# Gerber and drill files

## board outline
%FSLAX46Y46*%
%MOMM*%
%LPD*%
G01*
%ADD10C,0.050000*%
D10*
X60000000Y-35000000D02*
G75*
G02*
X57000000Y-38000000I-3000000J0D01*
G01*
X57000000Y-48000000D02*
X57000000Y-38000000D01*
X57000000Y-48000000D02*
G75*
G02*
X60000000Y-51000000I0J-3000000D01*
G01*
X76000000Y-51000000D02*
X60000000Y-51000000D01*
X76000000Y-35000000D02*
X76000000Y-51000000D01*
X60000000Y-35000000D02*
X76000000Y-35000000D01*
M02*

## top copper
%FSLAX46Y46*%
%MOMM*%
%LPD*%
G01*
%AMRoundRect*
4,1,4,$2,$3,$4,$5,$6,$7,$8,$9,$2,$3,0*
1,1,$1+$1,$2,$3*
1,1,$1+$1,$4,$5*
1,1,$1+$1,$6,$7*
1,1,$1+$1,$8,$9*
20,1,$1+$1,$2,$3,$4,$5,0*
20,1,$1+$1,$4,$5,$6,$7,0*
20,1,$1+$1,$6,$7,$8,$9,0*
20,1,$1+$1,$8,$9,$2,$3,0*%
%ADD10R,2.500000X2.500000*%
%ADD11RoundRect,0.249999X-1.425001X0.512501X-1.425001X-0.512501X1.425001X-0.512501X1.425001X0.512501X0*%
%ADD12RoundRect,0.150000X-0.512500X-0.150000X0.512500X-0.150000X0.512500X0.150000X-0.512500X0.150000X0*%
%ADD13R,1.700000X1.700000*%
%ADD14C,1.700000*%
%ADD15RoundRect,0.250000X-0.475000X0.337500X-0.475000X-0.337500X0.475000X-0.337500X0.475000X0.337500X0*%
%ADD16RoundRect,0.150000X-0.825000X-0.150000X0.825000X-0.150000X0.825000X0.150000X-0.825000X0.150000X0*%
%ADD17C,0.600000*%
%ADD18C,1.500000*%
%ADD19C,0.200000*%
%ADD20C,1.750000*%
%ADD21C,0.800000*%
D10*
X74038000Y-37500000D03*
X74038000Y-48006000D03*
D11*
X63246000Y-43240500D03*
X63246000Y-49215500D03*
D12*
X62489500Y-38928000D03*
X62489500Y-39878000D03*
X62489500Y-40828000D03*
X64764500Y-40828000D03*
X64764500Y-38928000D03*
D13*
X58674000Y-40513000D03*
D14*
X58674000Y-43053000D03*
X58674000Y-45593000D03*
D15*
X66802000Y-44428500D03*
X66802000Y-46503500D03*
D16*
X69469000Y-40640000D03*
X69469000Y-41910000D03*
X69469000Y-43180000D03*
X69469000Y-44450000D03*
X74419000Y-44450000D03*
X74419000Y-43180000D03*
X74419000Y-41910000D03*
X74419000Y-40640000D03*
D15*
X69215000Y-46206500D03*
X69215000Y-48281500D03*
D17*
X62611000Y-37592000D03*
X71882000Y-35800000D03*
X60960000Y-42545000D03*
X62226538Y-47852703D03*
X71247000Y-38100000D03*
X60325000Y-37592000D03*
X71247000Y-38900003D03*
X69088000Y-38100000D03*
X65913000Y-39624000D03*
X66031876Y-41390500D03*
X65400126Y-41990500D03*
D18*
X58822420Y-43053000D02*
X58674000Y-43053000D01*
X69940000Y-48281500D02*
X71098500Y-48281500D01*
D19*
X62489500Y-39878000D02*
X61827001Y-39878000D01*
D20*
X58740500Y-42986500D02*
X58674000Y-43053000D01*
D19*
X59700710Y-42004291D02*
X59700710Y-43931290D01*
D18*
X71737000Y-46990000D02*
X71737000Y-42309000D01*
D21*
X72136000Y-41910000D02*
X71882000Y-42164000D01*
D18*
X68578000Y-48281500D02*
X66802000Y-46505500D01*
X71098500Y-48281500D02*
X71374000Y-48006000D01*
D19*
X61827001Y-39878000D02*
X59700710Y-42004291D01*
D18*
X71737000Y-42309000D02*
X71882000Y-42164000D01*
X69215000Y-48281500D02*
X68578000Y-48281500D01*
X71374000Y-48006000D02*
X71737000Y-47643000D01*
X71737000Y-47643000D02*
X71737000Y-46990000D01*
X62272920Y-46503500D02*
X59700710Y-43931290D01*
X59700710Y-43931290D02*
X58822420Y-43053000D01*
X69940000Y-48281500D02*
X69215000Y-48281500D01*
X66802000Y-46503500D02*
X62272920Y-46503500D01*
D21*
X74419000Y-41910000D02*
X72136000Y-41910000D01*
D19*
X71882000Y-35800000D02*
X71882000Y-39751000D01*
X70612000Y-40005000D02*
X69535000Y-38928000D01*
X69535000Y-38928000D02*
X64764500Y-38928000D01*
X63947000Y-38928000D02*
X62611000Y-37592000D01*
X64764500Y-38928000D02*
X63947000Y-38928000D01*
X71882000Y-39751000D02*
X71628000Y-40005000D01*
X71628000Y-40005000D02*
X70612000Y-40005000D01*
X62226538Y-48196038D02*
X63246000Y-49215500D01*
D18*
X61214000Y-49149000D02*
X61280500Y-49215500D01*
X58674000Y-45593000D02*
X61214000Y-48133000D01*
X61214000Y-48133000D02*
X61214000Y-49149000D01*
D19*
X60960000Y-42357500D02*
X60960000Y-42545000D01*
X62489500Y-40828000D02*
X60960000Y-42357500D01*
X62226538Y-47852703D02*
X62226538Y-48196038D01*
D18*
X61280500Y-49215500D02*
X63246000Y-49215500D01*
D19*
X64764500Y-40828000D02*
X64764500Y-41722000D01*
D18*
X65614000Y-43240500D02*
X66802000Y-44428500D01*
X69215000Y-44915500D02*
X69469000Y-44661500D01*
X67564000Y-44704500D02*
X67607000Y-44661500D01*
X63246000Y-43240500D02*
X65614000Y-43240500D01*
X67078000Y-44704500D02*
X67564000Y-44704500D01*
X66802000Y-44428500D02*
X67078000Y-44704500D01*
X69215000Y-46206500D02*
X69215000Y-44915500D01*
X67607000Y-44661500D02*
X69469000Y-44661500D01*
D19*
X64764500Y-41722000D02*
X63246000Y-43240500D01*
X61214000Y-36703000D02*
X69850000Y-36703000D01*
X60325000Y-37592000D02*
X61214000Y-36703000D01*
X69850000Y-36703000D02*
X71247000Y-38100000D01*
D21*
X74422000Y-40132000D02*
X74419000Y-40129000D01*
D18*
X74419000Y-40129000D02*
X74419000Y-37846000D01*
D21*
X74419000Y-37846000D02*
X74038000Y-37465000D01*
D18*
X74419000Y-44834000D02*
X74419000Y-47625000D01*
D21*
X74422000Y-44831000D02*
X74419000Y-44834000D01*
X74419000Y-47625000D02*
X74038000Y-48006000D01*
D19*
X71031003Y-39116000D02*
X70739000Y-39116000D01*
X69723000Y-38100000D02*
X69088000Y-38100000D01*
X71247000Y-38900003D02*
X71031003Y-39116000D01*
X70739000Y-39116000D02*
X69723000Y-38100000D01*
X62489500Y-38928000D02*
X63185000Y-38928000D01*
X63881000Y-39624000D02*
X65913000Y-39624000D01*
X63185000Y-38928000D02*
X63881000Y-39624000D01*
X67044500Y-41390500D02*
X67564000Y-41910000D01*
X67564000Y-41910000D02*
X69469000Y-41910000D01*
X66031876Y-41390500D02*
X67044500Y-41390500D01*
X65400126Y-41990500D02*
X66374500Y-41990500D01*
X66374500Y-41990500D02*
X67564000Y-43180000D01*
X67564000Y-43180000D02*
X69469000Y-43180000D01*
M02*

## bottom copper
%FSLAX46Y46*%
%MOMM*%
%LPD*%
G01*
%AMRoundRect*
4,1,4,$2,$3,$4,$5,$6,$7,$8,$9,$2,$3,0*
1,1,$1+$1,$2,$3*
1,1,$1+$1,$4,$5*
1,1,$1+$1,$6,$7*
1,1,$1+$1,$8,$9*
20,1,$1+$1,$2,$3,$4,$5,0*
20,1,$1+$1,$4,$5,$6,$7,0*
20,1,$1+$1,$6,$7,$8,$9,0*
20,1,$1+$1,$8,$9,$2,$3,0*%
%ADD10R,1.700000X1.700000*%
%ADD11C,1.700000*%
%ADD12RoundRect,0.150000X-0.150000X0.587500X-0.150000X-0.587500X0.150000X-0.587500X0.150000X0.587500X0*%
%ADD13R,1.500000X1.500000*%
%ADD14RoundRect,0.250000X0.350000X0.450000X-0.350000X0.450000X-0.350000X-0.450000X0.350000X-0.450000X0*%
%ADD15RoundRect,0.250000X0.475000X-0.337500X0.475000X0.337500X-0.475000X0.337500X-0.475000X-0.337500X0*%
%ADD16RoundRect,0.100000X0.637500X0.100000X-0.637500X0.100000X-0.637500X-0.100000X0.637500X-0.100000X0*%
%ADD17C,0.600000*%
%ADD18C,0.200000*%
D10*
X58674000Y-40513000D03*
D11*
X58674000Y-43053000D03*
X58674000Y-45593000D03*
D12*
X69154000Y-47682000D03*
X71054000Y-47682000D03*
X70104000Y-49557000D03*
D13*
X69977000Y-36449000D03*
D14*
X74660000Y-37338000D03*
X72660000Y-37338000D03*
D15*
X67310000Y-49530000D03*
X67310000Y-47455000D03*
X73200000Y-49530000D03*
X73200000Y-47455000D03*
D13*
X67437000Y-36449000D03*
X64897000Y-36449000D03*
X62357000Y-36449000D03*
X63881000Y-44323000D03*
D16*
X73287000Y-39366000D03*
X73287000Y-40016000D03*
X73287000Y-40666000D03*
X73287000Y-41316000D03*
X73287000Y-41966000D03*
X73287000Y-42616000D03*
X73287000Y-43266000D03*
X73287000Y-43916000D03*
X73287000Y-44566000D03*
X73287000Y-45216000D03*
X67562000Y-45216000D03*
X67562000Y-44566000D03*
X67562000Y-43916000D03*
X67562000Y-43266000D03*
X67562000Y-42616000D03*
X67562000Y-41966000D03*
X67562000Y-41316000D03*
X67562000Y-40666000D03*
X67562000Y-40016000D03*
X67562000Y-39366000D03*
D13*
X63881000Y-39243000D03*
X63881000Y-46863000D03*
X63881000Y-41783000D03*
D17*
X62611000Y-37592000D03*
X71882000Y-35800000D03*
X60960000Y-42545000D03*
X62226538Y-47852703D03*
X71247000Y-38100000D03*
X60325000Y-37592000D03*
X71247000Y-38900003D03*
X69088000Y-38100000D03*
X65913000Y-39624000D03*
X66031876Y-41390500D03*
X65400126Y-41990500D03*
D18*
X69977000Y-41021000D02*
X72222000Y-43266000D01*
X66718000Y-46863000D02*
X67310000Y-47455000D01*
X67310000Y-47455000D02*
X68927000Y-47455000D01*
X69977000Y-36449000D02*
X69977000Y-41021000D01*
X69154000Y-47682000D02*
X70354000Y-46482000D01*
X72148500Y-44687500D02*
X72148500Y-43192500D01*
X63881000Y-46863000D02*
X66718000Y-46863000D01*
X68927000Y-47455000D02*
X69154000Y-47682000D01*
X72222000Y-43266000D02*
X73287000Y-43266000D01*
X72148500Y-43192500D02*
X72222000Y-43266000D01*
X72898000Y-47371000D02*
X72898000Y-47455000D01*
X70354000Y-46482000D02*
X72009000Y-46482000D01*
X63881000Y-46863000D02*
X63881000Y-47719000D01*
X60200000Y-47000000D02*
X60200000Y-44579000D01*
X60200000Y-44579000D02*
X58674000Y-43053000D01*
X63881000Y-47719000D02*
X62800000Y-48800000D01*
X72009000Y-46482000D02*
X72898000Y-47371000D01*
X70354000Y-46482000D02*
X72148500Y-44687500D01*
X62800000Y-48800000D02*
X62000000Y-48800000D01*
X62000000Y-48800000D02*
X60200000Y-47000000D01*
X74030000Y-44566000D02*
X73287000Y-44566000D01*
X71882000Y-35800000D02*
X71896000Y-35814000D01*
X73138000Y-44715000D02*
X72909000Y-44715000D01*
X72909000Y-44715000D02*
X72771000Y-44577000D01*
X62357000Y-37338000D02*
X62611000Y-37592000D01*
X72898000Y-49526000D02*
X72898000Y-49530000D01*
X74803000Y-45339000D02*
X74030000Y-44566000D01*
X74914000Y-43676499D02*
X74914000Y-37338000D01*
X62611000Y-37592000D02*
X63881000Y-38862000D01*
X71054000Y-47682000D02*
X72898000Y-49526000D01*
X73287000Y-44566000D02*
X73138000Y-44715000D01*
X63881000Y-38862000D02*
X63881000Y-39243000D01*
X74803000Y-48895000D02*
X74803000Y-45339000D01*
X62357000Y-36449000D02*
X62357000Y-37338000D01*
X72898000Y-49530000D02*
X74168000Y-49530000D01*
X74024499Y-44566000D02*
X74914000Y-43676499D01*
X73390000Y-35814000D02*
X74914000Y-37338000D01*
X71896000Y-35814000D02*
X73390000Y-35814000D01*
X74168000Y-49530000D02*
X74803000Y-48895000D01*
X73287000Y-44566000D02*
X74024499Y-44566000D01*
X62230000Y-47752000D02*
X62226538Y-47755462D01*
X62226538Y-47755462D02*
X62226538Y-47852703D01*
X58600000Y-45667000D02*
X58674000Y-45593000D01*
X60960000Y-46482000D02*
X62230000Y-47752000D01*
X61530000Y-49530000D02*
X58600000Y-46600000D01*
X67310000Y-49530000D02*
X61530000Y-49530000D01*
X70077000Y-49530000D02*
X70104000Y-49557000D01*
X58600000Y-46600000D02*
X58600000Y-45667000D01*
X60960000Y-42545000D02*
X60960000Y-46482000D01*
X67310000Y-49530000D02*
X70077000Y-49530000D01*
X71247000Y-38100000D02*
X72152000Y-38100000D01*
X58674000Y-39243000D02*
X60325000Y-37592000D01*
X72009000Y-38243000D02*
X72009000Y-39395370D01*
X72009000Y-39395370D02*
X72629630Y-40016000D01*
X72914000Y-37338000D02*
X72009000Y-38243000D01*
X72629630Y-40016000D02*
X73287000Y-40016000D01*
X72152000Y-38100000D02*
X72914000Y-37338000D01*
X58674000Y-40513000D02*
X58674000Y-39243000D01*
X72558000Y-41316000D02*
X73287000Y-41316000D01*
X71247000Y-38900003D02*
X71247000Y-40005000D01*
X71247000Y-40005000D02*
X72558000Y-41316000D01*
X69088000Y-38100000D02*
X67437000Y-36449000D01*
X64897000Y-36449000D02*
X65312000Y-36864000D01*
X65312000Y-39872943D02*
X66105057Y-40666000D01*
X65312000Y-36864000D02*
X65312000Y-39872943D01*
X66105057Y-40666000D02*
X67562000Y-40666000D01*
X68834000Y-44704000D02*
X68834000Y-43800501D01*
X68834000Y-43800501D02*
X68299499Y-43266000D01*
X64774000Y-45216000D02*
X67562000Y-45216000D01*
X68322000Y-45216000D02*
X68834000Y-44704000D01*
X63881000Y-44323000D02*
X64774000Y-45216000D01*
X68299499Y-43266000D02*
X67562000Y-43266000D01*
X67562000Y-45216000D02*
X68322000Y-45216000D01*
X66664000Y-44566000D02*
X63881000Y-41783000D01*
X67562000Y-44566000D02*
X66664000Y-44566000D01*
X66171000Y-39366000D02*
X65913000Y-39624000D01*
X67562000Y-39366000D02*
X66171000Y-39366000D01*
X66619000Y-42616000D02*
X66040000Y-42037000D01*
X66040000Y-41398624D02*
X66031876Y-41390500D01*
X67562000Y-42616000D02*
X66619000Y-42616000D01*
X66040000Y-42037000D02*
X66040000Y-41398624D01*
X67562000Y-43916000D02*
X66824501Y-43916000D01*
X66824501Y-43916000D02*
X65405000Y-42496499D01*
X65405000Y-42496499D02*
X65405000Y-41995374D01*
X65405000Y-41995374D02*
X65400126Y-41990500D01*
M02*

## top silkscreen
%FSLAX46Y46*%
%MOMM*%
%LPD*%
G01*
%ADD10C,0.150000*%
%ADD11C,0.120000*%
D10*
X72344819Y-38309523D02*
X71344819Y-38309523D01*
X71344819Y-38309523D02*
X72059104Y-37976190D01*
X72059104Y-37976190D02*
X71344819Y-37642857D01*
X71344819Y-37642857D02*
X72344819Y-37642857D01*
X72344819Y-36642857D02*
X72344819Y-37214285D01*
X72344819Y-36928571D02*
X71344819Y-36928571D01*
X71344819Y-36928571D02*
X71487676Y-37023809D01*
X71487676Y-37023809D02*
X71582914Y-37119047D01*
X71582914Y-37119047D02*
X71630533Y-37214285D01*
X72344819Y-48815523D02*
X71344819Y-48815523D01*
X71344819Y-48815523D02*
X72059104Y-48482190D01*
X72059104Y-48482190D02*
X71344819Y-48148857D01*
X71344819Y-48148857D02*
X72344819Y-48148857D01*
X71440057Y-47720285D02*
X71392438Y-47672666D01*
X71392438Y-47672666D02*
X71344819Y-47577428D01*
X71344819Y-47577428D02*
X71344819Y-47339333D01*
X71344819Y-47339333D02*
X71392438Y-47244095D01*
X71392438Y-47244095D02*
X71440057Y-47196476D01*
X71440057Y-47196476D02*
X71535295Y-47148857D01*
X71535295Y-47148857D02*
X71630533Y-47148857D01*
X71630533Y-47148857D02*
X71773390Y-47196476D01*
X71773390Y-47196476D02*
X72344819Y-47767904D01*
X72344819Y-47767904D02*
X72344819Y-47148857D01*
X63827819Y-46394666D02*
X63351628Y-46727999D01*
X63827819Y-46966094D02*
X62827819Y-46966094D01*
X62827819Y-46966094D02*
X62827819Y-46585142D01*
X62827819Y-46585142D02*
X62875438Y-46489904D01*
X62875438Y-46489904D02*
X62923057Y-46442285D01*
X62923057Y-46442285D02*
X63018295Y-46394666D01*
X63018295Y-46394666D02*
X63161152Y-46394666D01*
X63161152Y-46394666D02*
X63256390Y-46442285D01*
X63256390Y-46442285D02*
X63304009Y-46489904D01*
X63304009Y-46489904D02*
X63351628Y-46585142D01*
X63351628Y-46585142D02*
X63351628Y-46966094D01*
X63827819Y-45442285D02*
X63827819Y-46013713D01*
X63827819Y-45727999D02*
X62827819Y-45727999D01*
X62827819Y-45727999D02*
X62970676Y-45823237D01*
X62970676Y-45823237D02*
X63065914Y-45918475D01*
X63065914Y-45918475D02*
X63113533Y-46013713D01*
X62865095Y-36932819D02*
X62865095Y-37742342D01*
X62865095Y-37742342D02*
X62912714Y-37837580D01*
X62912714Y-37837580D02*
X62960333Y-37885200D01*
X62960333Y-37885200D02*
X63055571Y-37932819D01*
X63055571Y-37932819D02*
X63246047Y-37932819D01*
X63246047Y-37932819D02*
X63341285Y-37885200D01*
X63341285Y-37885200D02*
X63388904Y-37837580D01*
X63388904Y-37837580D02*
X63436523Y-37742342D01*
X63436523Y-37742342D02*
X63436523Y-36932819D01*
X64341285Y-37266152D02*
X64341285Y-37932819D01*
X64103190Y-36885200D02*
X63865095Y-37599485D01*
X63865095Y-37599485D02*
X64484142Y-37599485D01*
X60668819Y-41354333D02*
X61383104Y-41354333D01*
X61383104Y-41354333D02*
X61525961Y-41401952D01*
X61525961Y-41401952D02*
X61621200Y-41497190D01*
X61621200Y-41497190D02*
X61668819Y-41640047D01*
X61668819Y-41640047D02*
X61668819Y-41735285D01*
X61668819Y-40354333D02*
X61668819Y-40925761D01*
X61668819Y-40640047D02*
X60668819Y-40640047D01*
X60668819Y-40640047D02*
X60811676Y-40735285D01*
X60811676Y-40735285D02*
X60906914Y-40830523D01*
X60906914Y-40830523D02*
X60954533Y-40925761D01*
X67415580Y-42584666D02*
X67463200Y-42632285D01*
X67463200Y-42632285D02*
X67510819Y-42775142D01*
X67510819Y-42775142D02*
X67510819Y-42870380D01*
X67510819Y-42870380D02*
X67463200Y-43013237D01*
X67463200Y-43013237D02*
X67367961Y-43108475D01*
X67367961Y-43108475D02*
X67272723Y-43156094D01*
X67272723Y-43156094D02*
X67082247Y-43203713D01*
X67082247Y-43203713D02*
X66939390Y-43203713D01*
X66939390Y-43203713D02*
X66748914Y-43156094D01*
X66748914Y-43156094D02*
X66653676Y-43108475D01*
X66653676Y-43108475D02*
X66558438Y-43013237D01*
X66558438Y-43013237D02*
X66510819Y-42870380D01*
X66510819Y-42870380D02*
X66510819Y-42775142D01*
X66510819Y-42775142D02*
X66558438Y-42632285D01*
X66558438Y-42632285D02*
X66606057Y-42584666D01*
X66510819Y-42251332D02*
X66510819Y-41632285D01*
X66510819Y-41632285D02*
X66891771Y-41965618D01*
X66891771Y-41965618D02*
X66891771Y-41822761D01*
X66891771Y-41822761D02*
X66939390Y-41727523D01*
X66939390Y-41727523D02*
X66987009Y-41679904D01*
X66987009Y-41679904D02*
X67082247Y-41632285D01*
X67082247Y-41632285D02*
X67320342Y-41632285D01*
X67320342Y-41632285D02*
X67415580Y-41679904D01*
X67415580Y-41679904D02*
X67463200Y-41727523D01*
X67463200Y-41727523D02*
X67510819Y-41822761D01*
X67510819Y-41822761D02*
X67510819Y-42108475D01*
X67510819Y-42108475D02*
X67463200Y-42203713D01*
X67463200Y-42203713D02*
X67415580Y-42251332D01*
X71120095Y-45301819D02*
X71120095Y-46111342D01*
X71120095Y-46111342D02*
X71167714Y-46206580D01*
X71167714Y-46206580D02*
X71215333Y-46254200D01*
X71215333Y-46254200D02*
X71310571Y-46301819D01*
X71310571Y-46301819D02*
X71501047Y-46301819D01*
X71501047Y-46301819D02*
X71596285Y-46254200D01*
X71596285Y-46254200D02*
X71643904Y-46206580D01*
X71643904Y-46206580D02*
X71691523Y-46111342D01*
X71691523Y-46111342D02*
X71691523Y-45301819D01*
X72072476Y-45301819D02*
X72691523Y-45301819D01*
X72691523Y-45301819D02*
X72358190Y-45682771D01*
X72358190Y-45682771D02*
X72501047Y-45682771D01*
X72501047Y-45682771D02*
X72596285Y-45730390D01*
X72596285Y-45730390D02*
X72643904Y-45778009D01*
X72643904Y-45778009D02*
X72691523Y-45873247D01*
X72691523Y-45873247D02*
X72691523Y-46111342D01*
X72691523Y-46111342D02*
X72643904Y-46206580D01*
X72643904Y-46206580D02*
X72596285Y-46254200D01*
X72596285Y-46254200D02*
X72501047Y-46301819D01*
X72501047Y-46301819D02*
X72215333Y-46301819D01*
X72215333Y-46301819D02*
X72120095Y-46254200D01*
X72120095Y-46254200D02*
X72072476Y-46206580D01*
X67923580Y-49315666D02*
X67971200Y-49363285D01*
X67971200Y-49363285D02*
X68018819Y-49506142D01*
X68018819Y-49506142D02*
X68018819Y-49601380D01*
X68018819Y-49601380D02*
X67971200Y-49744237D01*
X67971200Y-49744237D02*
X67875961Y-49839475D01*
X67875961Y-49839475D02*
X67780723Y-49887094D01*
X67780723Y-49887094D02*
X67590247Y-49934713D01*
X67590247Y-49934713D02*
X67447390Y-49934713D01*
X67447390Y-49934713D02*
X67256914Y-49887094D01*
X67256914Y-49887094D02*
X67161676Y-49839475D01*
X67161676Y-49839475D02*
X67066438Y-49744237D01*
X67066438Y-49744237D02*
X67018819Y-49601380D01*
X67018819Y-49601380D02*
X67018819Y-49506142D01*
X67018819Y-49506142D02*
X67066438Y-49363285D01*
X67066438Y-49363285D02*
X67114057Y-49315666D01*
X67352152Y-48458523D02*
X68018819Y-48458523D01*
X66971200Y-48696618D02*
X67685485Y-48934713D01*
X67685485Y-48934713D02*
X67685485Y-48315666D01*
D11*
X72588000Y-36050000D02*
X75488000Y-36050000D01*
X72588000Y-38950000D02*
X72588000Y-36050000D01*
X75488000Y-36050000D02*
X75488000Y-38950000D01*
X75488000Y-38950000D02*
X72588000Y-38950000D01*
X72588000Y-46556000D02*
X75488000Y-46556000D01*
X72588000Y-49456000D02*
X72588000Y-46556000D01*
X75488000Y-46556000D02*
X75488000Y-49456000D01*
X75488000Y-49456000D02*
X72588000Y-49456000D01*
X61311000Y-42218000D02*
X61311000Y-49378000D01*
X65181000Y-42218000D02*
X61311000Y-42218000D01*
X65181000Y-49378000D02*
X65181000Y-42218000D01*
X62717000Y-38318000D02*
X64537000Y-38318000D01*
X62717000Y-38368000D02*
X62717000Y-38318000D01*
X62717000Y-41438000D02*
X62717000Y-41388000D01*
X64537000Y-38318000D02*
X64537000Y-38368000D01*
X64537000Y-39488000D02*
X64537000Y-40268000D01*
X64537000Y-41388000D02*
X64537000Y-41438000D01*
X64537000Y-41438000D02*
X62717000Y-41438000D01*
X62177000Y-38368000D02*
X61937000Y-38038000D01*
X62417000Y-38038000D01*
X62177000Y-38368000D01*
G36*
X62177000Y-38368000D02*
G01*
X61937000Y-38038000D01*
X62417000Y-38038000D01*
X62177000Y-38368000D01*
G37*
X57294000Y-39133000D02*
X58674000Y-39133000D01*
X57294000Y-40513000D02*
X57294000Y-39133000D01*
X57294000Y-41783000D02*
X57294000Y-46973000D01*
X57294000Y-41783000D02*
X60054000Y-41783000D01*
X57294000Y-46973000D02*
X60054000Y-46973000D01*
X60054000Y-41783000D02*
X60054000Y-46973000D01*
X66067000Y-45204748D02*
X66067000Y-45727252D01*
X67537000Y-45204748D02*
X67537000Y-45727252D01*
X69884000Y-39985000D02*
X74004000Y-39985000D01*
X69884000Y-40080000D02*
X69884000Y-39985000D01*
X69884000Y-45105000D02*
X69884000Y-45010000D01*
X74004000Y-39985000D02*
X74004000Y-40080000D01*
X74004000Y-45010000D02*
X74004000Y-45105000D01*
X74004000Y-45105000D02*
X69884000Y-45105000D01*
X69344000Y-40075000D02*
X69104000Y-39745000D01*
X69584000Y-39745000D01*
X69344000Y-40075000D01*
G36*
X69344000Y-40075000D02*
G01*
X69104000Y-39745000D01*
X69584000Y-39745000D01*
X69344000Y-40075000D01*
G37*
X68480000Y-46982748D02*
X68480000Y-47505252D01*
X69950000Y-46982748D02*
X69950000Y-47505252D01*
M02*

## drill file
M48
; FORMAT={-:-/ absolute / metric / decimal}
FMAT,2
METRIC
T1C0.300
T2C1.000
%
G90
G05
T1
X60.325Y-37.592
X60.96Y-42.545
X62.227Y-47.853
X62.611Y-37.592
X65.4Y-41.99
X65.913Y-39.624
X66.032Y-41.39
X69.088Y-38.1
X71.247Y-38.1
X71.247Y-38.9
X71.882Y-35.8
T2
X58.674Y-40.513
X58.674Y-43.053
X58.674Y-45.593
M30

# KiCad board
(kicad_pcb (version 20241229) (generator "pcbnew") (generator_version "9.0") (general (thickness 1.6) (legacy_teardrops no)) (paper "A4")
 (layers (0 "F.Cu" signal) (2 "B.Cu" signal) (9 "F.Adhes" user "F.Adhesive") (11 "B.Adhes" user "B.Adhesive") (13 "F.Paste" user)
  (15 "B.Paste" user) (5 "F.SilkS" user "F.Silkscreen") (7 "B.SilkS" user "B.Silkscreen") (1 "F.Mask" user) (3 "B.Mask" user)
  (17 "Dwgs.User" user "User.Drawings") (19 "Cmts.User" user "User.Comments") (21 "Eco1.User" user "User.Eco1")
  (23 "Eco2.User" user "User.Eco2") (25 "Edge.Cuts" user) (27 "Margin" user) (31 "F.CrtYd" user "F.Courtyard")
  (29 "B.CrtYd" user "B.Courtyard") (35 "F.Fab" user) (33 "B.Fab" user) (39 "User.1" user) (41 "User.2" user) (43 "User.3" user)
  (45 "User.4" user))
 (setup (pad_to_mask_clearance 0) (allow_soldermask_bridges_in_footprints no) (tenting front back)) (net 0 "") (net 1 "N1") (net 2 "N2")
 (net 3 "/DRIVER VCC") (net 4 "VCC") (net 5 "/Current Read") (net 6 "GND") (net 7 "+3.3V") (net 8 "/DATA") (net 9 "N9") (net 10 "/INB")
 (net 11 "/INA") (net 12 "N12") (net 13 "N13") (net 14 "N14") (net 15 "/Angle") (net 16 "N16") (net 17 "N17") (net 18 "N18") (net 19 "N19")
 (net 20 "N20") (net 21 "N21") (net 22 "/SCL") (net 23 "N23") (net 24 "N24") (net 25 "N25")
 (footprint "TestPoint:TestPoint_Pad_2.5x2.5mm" (layer "F.Cu") (at 74.038 37.5 90)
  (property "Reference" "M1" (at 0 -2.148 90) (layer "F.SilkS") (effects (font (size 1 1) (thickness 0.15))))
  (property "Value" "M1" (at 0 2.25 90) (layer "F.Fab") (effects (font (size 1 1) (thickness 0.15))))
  (fp_line (start 1.45 -1.45) (end 1.45 1.45) (stroke (width 0.12) (type solid)) (layer "F.SilkS"))
  (fp_line (start -1.45 -1.45) (end 1.45 -1.45) (stroke (width 0.12) (type solid)) (layer "F.SilkS"))
  (fp_line (start 1.45 1.45) (end -1.45 1.45) (stroke (width 0.12) (type solid)) (layer "F.SilkS"))
  (fp_line (start -1.45 1.45) (end -1.45 -1.45) (stroke (width 0.12) (type solid)) (layer "F.SilkS"))
  (pad "1" smd rect (at 0 0 90) (size 2.5 2.5) (layers "F.Cu" "F.Mask") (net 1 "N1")))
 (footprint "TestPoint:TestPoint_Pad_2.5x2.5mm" (layer "F.Cu") (at 74.038 48.006 90)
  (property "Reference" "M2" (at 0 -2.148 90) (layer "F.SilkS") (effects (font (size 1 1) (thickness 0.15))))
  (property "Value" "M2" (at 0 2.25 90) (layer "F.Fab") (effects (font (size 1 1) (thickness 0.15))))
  (fp_line (start 1.45 -1.45) (end 1.45 1.45) (stroke (width 0.12) (type solid)) (layer "F.SilkS"))
  (fp_line (start -1.45 -1.45) (end 1.45 -1.45) (stroke (width 0.12) (type solid)) (layer "F.SilkS"))
  (fp_line (start 1.45 1.45) (end -1.45 1.45) (stroke (width 0.12) (type solid)) (layer "F.SilkS"))
  (fp_line (start -1.45 1.45) (end -1.45 -1.45) (stroke (width 0.12) (type solid)) (layer "F.SilkS"))
  (pad "1" smd rect (at 0 0 90) (size 2.5 2.5) (layers "F.Cu" "F.Mask") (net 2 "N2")))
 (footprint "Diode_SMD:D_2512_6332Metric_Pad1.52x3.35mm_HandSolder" (layer "F.Cu") (at 63.246 46.228 -90)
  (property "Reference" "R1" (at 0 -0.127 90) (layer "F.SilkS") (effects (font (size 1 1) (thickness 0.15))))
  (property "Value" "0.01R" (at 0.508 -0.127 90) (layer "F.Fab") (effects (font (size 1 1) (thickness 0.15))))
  (fp_line (start -4.01 1.935) (end 3.15 1.935) (stroke (width 0.12) (type solid)) (layer "F.SilkS"))
  (fp_line (start -4.01 -1.935) (end -4.01 1.935) (stroke (width 0.12) (type solid)) (layer "F.SilkS"))
  (fp_line (start 3.15 -1.935) (end -4.01 -1.935) (stroke (width 0.12) (type solid)) (layer "F.SilkS"))
  (pad "1" smd roundrect (at -2.9875 0 270) (size 1.525 3.35) (layers "F.Cu" "F.Mask" "F.Paste") (roundrect_rratio 0.163934)
   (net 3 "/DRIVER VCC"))
  (pad "2" smd roundrect (at 2.9875 0 270) (size 1.525 3.35) (layers "F.Cu" "F.Mask" "F.Paste") (roundrect_rratio 0.163934) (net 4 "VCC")))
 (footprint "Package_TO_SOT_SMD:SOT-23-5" (layer "F.Cu") (at 63.627 39.878)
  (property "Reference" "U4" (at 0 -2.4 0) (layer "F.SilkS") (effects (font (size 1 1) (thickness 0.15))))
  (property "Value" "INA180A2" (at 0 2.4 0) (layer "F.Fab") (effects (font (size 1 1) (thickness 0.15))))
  (fp_line (start -0.91 -1.56) (end 0.91 -1.56) (stroke (width 0.12) (type solid)) (layer "F.SilkS"))
  (fp_line (start -0.91 -1.51) (end -0.91 -1.56) (stroke (width 0.12) (type solid)) (layer "F.SilkS"))
  (fp_line (start -0.91 1.56) (end -0.91 1.51) (stroke (width 0.12) (type solid)) (layer "F.SilkS"))
  (fp_line (start 0.91 -1.56) (end 0.91 -1.51) (stroke (width 0.12) (type solid)) (layer "F.SilkS"))
  (fp_line (start 0.91 -0.39) (end 0.91 0.39) (stroke (width 0.12) (type solid)) (layer "F.SilkS"))
  (fp_line (start 0.91 1.51) (end 0.91 1.56) (stroke (width 0.12) (type solid)) (layer "F.SilkS"))
  (fp_line (start 0.91 1.56) (end -0.91 1.56) (stroke (width 0.12) (type solid)) (layer "F.SilkS"))
  (fp_poly (pts (xy -1.45 -1.51) (xy -1.69 -1.84) (xy -1.21 -1.84)) (stroke (width 0.12) (type solid)) (fill yes) (layer "F.SilkS"))
  (pad "1" smd roundrect (at -1.1375 -0.95) (size 1.325 0.6) (layers "F.Cu" "F.Mask" "F.Paste") (roundrect_rratio 0.25)
   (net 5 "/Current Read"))
  (pad "2" smd roundrect (at -1.1375 0) (size 1.325 0.6) (layers "F.Cu" "F.Mask" "F.Paste") (roundrect_rratio 0.25) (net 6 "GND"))
  (pad "3" smd roundrect (at -1.1375 0.95) (size 1.325 0.6) (layers "F.Cu" "F.Mask" "F.Paste") (roundrect_rratio 0.25) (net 4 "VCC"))
  (pad "4" smd roundrect (at 1.1375 0.95) (size 1.325 0.6) (layers "F.Cu" "F.Mask" "F.Paste") (roundrect_rratio 0.25) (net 3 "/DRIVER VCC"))
  (pad "5" smd roundrect (at 1.1375 -0.95) (size 1.325 0.6) (layers "F.Cu" "F.Mask" "F.Paste") (roundrect_rratio 0.25) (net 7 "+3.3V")))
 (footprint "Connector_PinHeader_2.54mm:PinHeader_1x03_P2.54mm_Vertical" (layer "F.Cu") (at 58.674 40.513)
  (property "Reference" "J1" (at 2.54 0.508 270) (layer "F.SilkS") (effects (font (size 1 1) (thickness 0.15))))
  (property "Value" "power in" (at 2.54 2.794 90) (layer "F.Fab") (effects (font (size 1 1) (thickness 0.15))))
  (fp_line (start -1.38 -1.38) (end 0 -1.38) (stroke (width 0.12) (type solid)) (layer "F.SilkS"))
  (fp_line (start -1.38 0) (end -1.38 -1.38) (stroke (width 0.12) (type solid)) (layer "F.SilkS"))
  (fp_line (start -1.38 1.27) (end -1.38 6.46) (stroke (width 0.12) (type solid)) (layer "F.SilkS"))
  (fp_line (start -1.38 1.27) (end 1.38 1.27) (stroke (width 0.12) (type solid)) (layer "F.SilkS"))
  (fp_line (start -1.38 6.46) (end 1.38 6.46) (stroke (width 0.12) (type solid)) (layer "F.SilkS"))
  (fp_line (start 1.38 1.27) (end 1.38 6.46) (stroke (width 0.12) (type solid)) (layer "F.SilkS"))
  (pad "1" thru_hole rect (at 0 0) (size 1.7 1.7) (drill 1) (layers "*.Cu" "*.Mask") (remove_unused_layers no) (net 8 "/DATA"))
  (pad "2" thru_hole circle (at 0 2.54) (size 1.7 1.7) (drill 1) (layers "*.Cu" "*.Mask") (remove_unused_layers no) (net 6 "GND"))
  (pad "3" thru_hole circle (at 0 5.08) (size 1.7 1.7) (drill 1) (layers "*.Cu" "*.Mask") (remove_unused_layers no) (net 4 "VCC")))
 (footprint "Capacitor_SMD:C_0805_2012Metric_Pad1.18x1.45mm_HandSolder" (layer "F.Cu") (at 66.802 45.466 -90)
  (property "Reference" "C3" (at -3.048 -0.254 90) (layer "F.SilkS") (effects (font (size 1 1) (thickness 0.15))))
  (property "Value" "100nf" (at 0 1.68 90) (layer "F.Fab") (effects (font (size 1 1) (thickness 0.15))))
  (fp_line (start -0.261252 0.735) (end 0.261252 0.735) (stroke (width 0.12) (type solid)) (layer "F.SilkS"))
  (fp_line (start -0.261252 -0.735) (end 0.261252 -0.735) (stroke (width 0.12) (type solid)) (layer "F.SilkS"))
  (pad "1" smd roundrect (at -1.0375 0 270) (size 1.175 1.45) (layers "F.Cu" "F.Mask" "F.Paste") (roundrect_rratio 0.212766)
   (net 3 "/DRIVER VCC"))
  (pad "2" smd roundrect (at 1.0375 0 270) (size 1.175 1.45) (layers "F.Cu" "F.Mask" "F.Paste") (roundrect_rratio 0.212766) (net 6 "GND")))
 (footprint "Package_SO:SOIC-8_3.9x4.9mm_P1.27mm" (layer "F.Cu") (at 71.944 42.545)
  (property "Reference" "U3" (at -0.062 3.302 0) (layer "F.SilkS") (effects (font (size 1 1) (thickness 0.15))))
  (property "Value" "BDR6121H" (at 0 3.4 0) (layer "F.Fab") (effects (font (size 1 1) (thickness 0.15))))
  (fp_line (start -2.06 -2.56) (end 2.06 -2.56) (stroke (width 0.12) (type solid)) (layer "F.SilkS"))
  (fp_line (start -2.06 -2.465) (end -2.06 -2.56) (stroke (width 0.12) (type solid)) (layer "F.SilkS"))
  (fp_line (start -2.06 2.56) (end -2.06 2.465) (stroke (width 0.12) (type solid)) (layer "F.SilkS"))
  (fp_line (start 2.06 -2.56) (end 2.06 -2.465) (stroke (width 0.12) (type solid)) (layer "F.SilkS"))
  (fp_line (start 2.06 2.465) (end 2.06 2.56) (stroke (width 0.12) (type solid)) (layer "F.SilkS"))
  (fp_line (start 2.06 2.56) (end -2.06 2.56) (stroke (width 0.12) (type solid)) (layer "F.SilkS"))
  (fp_poly (pts (xy -2.6 -2.47) (xy -2.84 -2.8) (xy -2.36 -2.8)) (stroke (width 0.12) (type solid)) (fill yes) (layer "F.SilkS"))
  (pad "1" smd roundrect (at -2.475 -1.905) (size 1.95 0.6) (layers "F.Cu" "F.Mask" "F.Paste") (roundrect_rratio 0.25) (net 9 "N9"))
  (pad "2" smd roundrect (at -2.475 -0.635) (size 1.95 0.6) (layers "F.Cu" "F.Mask" "F.Paste") (roundrect_rratio 0.25) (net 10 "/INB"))
  (pad "3" smd roundrect (at -2.475 0.635) (size 1.95 0.6) (layers "F.Cu" "F.Mask" "F.Paste") (roundrect_rratio 0.25) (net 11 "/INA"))
  (pad "4" smd roundrect (at -2.475 1.905) (size 1.95 0.6) (layers "F.Cu" "F.Mask" "F.Paste") (roundrect_rratio 0.25) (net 3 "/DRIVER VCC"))
  (pad "5" smd roundrect (at 2.475 1.905) (size 1.95 0.6) (layers "F.Cu" "F.Mask" "F.Paste") (roundrect_rratio 0.25) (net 2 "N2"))
  (pad "6" smd roundrect (at 2.475 0.635) (size 1.95 0.6) (layers "F.Cu" "F.Mask" "F.Paste") (roundrect_rratio 0.25) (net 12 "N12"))
  (pad "7" smd roundrect (at 2.475 -0.635) (size 1.95 0.6) (layers "F.Cu" "F.Mask" "F.Paste") (roundrect_rratio 0.25) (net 6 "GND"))
  (pad "8" smd roundrect (at 2.475 -1.905) (size 1.95 0.6) (layers "F.Cu" "F.Mask" "F.Paste") (roundrect_rratio 0.25) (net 1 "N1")))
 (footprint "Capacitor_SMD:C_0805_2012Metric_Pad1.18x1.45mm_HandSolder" (layer "F.Cu") (at 69.215 47.244 -90)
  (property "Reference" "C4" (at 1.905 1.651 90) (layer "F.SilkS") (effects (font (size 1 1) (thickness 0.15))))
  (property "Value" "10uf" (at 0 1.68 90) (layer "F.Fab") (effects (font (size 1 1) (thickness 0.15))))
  (fp_line (start -0.261252 0.735) (end 0.261252 0.735) (stroke (width 0.12) (type solid)) (layer "F.SilkS"))
  (fp_line (start -0.261252 -0.735) (end 0.261252 -0.735) (stroke (width 0.12) (type solid)) (layer "F.SilkS"))
  (pad "1" smd roundrect (at -1.0375 0 270) (size 1.175 1.45) (layers "F.Cu" "F.Mask" "F.Paste") (roundrect_rratio 0.212766)
   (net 3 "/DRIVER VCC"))
  (pad "2" smd roundrect (at 1.0375 0 270) (size 1.175 1.45) (layers "F.Cu" "F.Mask" "F.Paste") (roundrect_rratio 0.212766) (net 6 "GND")))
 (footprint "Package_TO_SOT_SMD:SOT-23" (layer "B.Cu") (at 70.104 48.6195 -90)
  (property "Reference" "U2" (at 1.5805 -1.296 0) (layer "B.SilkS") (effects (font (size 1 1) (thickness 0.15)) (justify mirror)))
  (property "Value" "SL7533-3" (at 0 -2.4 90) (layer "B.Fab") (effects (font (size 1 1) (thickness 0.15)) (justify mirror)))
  (pad "1" smd roundrect (at -0.9375 0.95 270) (size 1.475 0.6) (layers "B.Cu" "B.Mask" "B.Paste") (roundrect_rratio 0.25) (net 6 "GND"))
  (pad "2" smd roundrect (at -0.9375 -0.95 270) (size 1.475 0.6) (layers "B.Cu" "B.Mask" "B.Paste") (roundrect_rratio 0.25) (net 7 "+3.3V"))
  (pad "3" smd roundrect (at 0.9375 0 270) (size 1.475 0.6) (layers "B.Cu" "B.Mask" "B.Paste") (roundrect_rratio 0.25) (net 4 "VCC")))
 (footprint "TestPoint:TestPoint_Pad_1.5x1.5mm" (layer "B.Cu") (at 69.977 36.449 90)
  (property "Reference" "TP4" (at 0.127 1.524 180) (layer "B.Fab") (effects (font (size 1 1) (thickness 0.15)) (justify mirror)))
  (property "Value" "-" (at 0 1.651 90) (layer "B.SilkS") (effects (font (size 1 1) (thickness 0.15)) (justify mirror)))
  (pad "1" smd rect (at 0 0 90) (size 1.5 1.5) (layers "B.Cu" "B.Mask") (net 6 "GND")))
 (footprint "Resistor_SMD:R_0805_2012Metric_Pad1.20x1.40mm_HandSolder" (layer "B.Cu") (at 73.66 37.338 180)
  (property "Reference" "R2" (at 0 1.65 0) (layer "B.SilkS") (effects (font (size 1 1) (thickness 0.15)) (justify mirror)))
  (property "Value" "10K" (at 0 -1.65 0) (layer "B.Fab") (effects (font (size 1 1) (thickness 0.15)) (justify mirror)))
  (pad "1" smd roundrect (at -1 0 180) (size 1.2 1.4) (layers "B.Cu" "B.Mask" "B.Paste") (roundrect_rratio 0.208333) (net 7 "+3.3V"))
  (pad "2" smd roundrect (at 1 0 180) (size 1.2 1.4) (layers "B.Cu" "B.Mask" "B.Paste") (roundrect_rratio 0.208333) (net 8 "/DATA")))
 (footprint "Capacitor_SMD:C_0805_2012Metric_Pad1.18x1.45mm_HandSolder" (layer "B.Cu") (at 67.31 48.4925 90)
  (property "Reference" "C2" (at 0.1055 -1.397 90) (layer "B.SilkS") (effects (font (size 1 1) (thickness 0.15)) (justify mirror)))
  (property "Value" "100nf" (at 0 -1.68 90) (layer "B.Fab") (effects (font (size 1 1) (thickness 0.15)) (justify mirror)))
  (pad "1" smd roundrect (at -1.0375 0 90) (size 1.175 1.45) (layers "B.Cu" "B.Mask" "B.Paste") (roundrect_rratio 0.212766) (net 4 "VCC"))
  (pad "2" smd roundrect (at 1.0375 0 90) (size 1.175 1.45) (layers "B.Cu" "B.Mask" "B.Paste") (roundrect_rratio 0.212766) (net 6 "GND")))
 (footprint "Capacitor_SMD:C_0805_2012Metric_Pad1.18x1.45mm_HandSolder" (layer "B.Cu") (at 73.2 48.4925 90)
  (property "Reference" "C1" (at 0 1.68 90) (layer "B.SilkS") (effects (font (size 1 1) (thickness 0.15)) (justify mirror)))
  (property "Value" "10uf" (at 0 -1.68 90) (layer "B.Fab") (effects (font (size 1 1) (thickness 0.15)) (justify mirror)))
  (pad "1" smd roundrect (at -1.0375 0 90) (size 1.175 1.45) (layers "B.Cu" "B.Mask" "B.Paste") (roundrect_rratio 0.212766) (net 7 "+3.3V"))
  (pad "2" smd roundrect (at 1.0375 0 90) (size 1.175 1.45) (layers "B.Cu" "B.Mask" "B.Paste") (roundrect_rratio 0.212766) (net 6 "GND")))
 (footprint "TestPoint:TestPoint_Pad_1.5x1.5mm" (layer "B.Cu") (at 67.437 36.449 90)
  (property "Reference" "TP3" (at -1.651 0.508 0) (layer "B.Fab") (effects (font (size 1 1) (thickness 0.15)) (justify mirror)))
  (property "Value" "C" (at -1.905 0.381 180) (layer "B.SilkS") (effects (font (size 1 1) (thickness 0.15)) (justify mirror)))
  (pad "1" smd rect (at 0 0 90) (size 1.5 1.5) (layers "B.Cu" "B.Mask") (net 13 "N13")))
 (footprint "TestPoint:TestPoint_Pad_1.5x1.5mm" (layer "B.Cu") (at 64.897 36.449 90)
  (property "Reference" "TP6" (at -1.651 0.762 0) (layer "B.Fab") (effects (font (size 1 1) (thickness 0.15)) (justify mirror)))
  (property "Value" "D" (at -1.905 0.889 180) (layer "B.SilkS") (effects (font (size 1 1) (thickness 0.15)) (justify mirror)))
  (pad "1" smd rect (at 0 0 90) (size 1.5 1.5) (layers "B.Cu" "B.Mask") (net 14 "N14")))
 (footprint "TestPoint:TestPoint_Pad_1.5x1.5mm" (layer "B.Cu") (at 62.357 36.449 -90)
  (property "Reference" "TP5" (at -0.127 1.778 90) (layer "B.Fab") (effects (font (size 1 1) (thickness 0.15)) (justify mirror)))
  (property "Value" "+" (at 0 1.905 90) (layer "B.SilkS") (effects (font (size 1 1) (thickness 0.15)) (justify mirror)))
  (pad "1" smd rect (at 0 0 270) (size 1.5 1.5) (layers "B.Cu" "B.Mask") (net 7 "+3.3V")))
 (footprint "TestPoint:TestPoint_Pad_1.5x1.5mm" (layer "B.Cu") (at 63.881 44.323 -90)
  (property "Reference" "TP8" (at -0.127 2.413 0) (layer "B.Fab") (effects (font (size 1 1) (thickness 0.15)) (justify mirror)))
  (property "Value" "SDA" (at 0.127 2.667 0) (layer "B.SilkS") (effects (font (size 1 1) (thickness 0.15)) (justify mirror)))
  (pad "1" smd rect (at 0 0 270) (size 1.5 1.5) (layers "B.Cu" "B.Mask") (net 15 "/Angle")))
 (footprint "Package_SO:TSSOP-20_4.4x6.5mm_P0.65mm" (layer "B.Cu") (at 70.4245 42.291 180)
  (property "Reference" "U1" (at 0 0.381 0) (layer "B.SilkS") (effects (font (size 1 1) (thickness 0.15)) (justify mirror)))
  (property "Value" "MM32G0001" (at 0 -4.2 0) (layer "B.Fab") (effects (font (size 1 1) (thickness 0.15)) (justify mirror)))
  (pad "1" smd roundrect (at -2.8625 2.925 180) (size 1.475 0.4) (layers "B.Cu" "B.Mask" "B.Paste") (roundrect_rratio 0.25) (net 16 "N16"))
  (pad "2" smd roundrect (at -2.8625 2.275 180) (size 1.475 0.4) (layers "B.Cu" "B.Mask" "B.Paste") (roundrect_rratio 0.25) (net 8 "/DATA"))
  (pad "3" smd roundrect (at -2.8625 1.625 180) (size 1.475 0.4) (layers "B.Cu" "B.Mask" "B.Paste") (roundrect_rratio 0.25) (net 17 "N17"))
  (pad "4" smd roundrect (at -2.8625 0.975 180) (size 1.475 0.4) (layers "B.Cu" "B.Mask" "B.Paste") (roundrect_rratio 0.25) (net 13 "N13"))
  (pad "5" smd roundrect (at -2.8625 0.325 180) (size 1.475 0.4) (layers "B.Cu" "B.Mask" "B.Paste") (roundrect_rratio 0.25) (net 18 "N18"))
  (pad "6" smd roundrect (at -2.8625 -0.325 180) (size 1.475 0.4) (layers "B.Cu" "B.Mask" "B.Paste") (roundrect_rratio 0.25) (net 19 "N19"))
  (pad "7" smd roundrect (at -2.8625 -0.975 180) (size 1.475 0.4) (layers "B.Cu" "B.Mask" "B.Paste") (roundrect_rratio 0.25) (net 6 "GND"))
  (pad "8" smd roundrect (at -2.8625 -1.625 180) (size 1.475 0.4) (layers "B.Cu" "B.Mask" "B.Paste") (roundrect_rratio 0.25) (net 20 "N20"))
  (pad "9" smd roundrect (at -2.8625 -2.275 180) (size 1.475 0.4) (layers "B.Cu" "B.Mask" "B.Paste") (roundrect_rratio 0.25) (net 7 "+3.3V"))
  (pad "10" smd roundrect (at -2.8625 -2.925 180) (size 1.475 0.4) (layers "B.Cu" "B.Mask" "B.Paste") (roundrect_rratio 0.25) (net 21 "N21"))
  (pad "11" smd roundrect (at 2.8625 -2.925 180) (size 1.475 0.4) (layers "B.Cu" "B.Mask" "B.Paste") (roundrect_rratio 0.25)
   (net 15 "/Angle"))
  (pad "12" smd roundrect (at 2.8625 -2.275 180) (size 1.475 0.4) (layers "B.Cu" "B.Mask" "B.Paste") (roundrect_rratio 0.25) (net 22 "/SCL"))
  (pad "13" smd roundrect (at 2.8625 -1.625 180) (size 1.475 0.4) (layers "B.Cu" "B.Mask" "B.Paste") (roundrect_rratio 0.25) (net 11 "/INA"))
  (pad "14" smd roundrect (at 2.8625 -0.975 180) (size 1.475 0.4) (layers "B.Cu" "B.Mask" "B.Paste") (roundrect_rratio 0.25)
   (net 15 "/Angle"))
  (pad "15" smd roundrect (at 2.8625 -0.325 180) (size 1.475 0.4) (layers "B.Cu" "B.Mask" "B.Paste") (roundrect_rratio 0.25) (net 10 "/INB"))
  (pad "16" smd roundrect (at 2.8625 0.325 180) (size 1.475 0.4) (layers "B.Cu" "B.Mask" "B.Paste") (roundrect_rratio 0.25) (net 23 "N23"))
  (pad "17" smd roundrect (at 2.8625 0.975 180) (size 1.475 0.4) (layers "B.Cu" "B.Mask" "B.Paste") (roundrect_rratio 0.25) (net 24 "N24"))
  (pad "18" smd roundrect (at 2.8625 1.625 180) (size 1.475 0.4) (layers "B.Cu" "B.Mask" "B.Paste") (roundrect_rratio 0.25) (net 14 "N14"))
  (pad "19" smd roundrect (at 2.8625 2.275 180) (size 1.475 0.4) (layers "B.Cu" "B.Mask" "B.Paste") (roundrect_rratio 0.25) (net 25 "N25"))
  (pad "20" smd roundrect (at 2.8625 2.925 180) (size 1.475 0.4) (layers "B.Cu" "B.Mask" "B.Paste") (roundrect_rratio 0.25)
   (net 5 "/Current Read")))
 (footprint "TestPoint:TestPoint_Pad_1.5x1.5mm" (layer "B.Cu") (at 63.881 39.243 -90)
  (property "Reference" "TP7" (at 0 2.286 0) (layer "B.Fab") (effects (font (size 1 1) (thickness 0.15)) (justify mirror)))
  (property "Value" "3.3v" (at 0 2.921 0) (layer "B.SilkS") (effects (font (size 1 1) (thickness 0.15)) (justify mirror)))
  (pad "1" smd rect (at 0 0 270) (size 1.5 1.5) (layers "B.Cu" "B.Mask") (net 7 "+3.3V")))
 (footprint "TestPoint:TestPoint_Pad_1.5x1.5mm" (layer "B.Cu") (at 63.881 46.863 -90)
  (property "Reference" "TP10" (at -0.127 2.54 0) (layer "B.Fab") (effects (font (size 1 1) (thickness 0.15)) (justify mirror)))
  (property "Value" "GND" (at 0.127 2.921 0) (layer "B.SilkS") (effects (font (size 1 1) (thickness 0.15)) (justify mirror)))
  (pad "1" smd rect (at 0 0 270) (size 1.5 1.5) (layers "B.Cu" "B.Mask") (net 6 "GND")))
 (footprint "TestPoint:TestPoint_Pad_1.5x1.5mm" (layer "B.Cu") (at 63.881 41.783 -90)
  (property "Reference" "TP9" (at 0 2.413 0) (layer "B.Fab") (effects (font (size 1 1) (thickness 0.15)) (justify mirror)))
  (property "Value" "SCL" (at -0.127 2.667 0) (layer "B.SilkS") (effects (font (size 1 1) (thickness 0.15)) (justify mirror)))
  (pad "1" smd rect (at 0 0 270) (size 1.5 1.5) (layers "B.Cu" "B.Mask") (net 22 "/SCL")))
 (gr_arc (start 60 35) (mid 59.12132 37.12132) (end 57 38) (stroke (width 0.05) (type default)) (layer "Edge.Cuts"))
 (gr_line (start 57 48) (end 57 38) (stroke (width 0.05) (type default)) (layer "Edge.Cuts"))
 (gr_arc (start 57 48) (mid 59.12132 48.87868) (end 60 51) (stroke (width 0.05) (type default)) (layer "Edge.Cuts"))
 (gr_line (start 76 51) (end 60 51) (stroke (width 0.05) (type default)) (layer "Edge.Cuts"))
 (gr_line (start 76 35) (end 76 51) (stroke (width 0.05) (type default)) (layer "Edge.Cuts"))
 (gr_line (start 60 35) (end 76 35) (stroke (width 0.05) (type default)) (layer "Edge.Cuts"))
 (segment (start 58.82242 43.053) (end 58.674 43.053) (width 1.5) (layer "F.Cu") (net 6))
 (segment (start 69.94 48.2815) (end 71.0985 48.2815) (width 1.5) (layer "F.Cu") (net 6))
 (segment (start 62.4895 39.878) (end 61.827001 39.878) (width 0.2) (layer "F.Cu") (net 6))
 (segment (start 58.7405 42.9865) (end 58.674 43.053) (width 1.75) (layer "F.Cu") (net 6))
 (segment (start 59.70071 42.004291) (end 59.70071 43.93129) (width 0.2) (layer "F.Cu") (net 6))
 (segment (start 71.737 46.99) (end 71.737 42.309) (width 1.5) (layer "F.Cu") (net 6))
 (segment (start 72.136 41.91) (end 71.882 42.164) (width 0.8) (layer "F.Cu") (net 6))
 (segment (start 68.578 48.2815) (end 66.802 46.5055) (width 1.5) (layer "F.Cu") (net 6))
 (segment (start 71.0985 48.2815) (end 71.374 48.006) (width 1.5) (layer "F.Cu") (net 6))
 (segment (start 61.827001 39.878) (end 59.70071 42.004291) (width 0.2) (layer "F.Cu") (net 6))
 (segment (start 71.737 42.309) (end 71.882 42.164) (width 1.5) (layer "F.Cu") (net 6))
 (segment (start 69.215 48.2815) (end 68.578 48.2815) (width 1.5) (layer "F.Cu") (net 6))
 (segment (start 71.374 48.006) (end 71.737 47.643) (width 1.5) (layer "F.Cu") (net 6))
 (segment (start 71.737 47.643) (end 71.737 46.99) (width 1.5) (layer "F.Cu") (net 6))
 (segment (start 62.27292 46.5035) (end 59.70071 43.93129) (width 1.5) (layer "F.Cu") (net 6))
 (segment (start 59.70071 43.93129) (end 58.82242 43.053) (width 1.5) (layer "F.Cu") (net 6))
 (segment (start 69.94 48.2815) (end 69.215 48.2815) (width 1.5) (layer "F.Cu") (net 6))
 (segment (start 66.802 46.5035) (end 62.27292 46.5035) (width 1.5) (layer "F.Cu") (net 6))
 (segment (start 74.419 41.91) (end 72.136 41.91) (width 0.8) (layer "F.Cu") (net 6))
 (segment (start 69.977 41.021) (end 72.222 43.266) (width 0.2) (layer "B.Cu") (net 6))
 (segment (start 66.718 46.863) (end 67.31 47.455) (width 0.2) (layer "B.Cu") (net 6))
 (segment (start 67.31 47.455) (end 68.927 47.455) (width 0.2) (layer "B.Cu") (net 6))
 (segment (start 69.977 36.449) (end 69.977 41.021) (width 0.2) (layer "B.Cu") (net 6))
 (segment (start 69.154 47.682) (end 70.354 46.482) (width 0.2) (layer "B.Cu") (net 6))
 (segment (start 72.1485 44.6875) (end 72.1485 43.1925) (width 0.2) (layer "B.Cu") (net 6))
 (segment (start 63.881 46.863) (end 66.718 46.863) (width 0.2) (layer "B.Cu") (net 6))
 (segment (start 68.927 47.455) (end 69.154 47.682) (width 0.2) (layer "B.Cu") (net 6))
 (segment (start 72.222 43.266) (end 73.287 43.266) (width 0.2) (layer "B.Cu") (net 6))
 (segment (start 72.1485 43.1925) (end 72.222 43.266) (width 0.2) (layer "B.Cu") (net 6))
 (segment (start 72.898 47.371) (end 72.898 47.455) (width 0.2) (layer "B.Cu") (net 6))
 (segment (start 70.354 46.482) (end 72.009 46.482) (width 0.2) (layer "B.Cu") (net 6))
 (segment (start 63.881 46.863) (end 63.881 47.719) (width 0.2) (layer "B.Cu") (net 6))
 (segment (start 60.2 47) (end 60.2 44.579) (width 0.2) (layer "B.Cu") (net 6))
 (segment (start 60.2 44.579) (end 58.674 43.053) (width 0.2) (layer "B.Cu") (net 6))
 (segment (start 63.881 47.719) (end 62.8 48.8) (width 0.2) (layer "B.Cu") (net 6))
 (segment (start 72.009 46.482) (end 72.898 47.371) (width 0.2) (layer "B.Cu") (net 6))
 (segment (start 70.354 46.482) (end 72.1485 44.6875) (width 0.2) (layer "B.Cu") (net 6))
 (segment (start 62.8 48.8) (end 62 48.8) (width 0.2) (layer "B.Cu") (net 6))
 (segment (start 62 48.8) (end 60.2 47) (width 0.2) (layer "B.Cu") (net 6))
 (segment (start 71.882 35.8) (end 71.882 39.751) (width 0.2) (layer "F.Cu") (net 7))
 (segment (start 70.612 40.005) (end 69.535 38.928) (width 0.2) (layer "F.Cu") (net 7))
 (segment (start 69.535 38.928) (end 64.7645 38.928) (width 0.2) (layer "F.Cu") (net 7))
 (segment (start 63.947 38.928) (end 62.611 37.592) (width 0.2) (layer "F.Cu") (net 7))
 (segment (start 64.7645 38.928) (end 63.947 38.928) (width 0.2) (layer "F.Cu") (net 7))
 (segment (start 71.882 39.751) (end 71.628 40.005) (width 0.2) (layer "F.Cu") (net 7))
 (segment (start 71.628 40.005) (end 70.612 40.005) (width 0.2) (layer "F.Cu") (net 7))
 (via (at 62.611 37.592) (size 0.6) (drill 0.3) (layers "F.Cu" "B.Cu") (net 7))
 (via (at 71.882 35.8) (size 0.6) (drill 0.3) (layers "F.Cu" "B.Cu") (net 7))
 (segment (start 74.03 44.566) (end 73.287 44.566) (width 0.2) (layer "B.Cu") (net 7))
 (segment (start 71.882 35.8) (end 71.896 35.814) (width 0.2) (layer "B.Cu") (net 7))
 (segment (start 73.138 44.715) (end 72.909 44.715) (width 0.2) (layer "B.Cu") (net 7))
 (segment (start 72.909 44.715) (end 72.771 44.577) (width 0.2) (layer "B.Cu") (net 7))
 (segment (start 62.357 37.338) (end 62.611 37.592) (width 0.2) (layer "B.Cu") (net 7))
 (segment (start 72.898 49.526) (end 72.898 49.53) (width 0.2) (layer "B.Cu") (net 7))
 (segment (start 74.803 45.339) (end 74.03 44.566) (width 0.2) (layer "B.Cu") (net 7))
 (segment (start 74.914 43.676499) (end 74.914 37.338) (width 0.2) (layer "B.Cu") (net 7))
 (segment (start 62.611 37.592) (end 63.881 38.862) (width 0.2) (layer "B.Cu") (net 7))
 (segment (start 71.054 47.682) (end 72.898 49.526) (width 0.2) (layer "B.Cu") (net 7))
 (segment (start 73.287 44.566) (end 73.138 44.715) (width 0.2) (layer "B.Cu") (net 7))
 (segment (start 63.881 38.862) (end 63.881 39.243) (width 0.2) (layer "B.Cu") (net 7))
 (segment (start 74.803 48.895) (end 74.803 45.339) (width 0.2) (layer "B.Cu") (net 7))
 (segment (start 62.357 36.449) (end 62.357 37.338) (width 0.2) (layer "B.Cu") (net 7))
 (segment (start 72.898 49.53) (end 74.168 49.53) (width 0.2) (layer "B.Cu") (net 7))
 (segment (start 74.024499 44.566) (end 74.914 43.676499) (width 0.2) (layer "B.Cu") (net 7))
 (segment (start 73.39 35.814) (end 74.914 37.338) (width 0.2) (layer "B.Cu") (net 7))
 (segment (start 71.896 35.814) (end 73.39 35.814) (width 0.2) (layer "B.Cu") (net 7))
 (segment (start 74.168 49.53) (end 74.803 48.895) (width 0.2) (layer "B.Cu") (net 7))
 (segment (start 73.287 44.566) (end 74.024499 44.566) (width 0.2) (layer "B.Cu") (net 7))
 (segment (start 62.226538 48.196038) (end 63.246 49.2155) (width 0.2) (layer "F.Cu") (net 4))
 (segment (start 61.214 49.149) (end 61.2805 49.2155) (width 1.5) (layer "F.Cu") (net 4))
 (segment (start 58.674 45.593) (end 61.214 48.133) (width 1.5) (layer "F.Cu") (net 4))
 (segment (start 61.214 48.133) (end 61.214 49.149) (width 1.5) (layer "F.Cu") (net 4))
 (segment (start 60.96 42.3575) (end 60.96 42.545) (width 0.2) (layer "F.Cu") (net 4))
 (segment (start 62.4895 40.828) (end 60.96 42.3575) (width 0.2) (layer "F.Cu") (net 4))
 (segment (start 62.226538 47.852703) (end 62.226538 48.196038) (width 0.2) (layer "F.Cu") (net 4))
 (segment (start 61.2805 49.2155) (end 63.246 49.2155) (width 1.5) (layer "F.Cu") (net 4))
 (via (at 60.96 42.545) (size 0.6) (drill 0.3) (layers "F.Cu" "B.Cu") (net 4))
 (via (at 62.226538 47.852703) (size 0.6) (drill 0.3) (layers "F.Cu" "B.Cu") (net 4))
 (segment (start 62.23 47.752) (end 62.226538 47.755462) (width 0.2) (layer "B.Cu") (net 4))
 (segment (start 62.226538 47.755462) (end 62.226538 47.852703) (width 0.2) (layer "B.Cu") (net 4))
 (segment (start 58.6 45.667) (end 58.674 45.593) (width 0.2) (layer "B.Cu") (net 4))
 (segment (start 60.96 46.482) (end 62.23 47.752) (width 0.2) (layer "B.Cu") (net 4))
 (segment (start 61.53 49.53) (end 58.6 46.6) (width 0.2) (layer "B.Cu") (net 4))
 (segment (start 67.31 49.53) (end 61.53 49.53) (width 0.2) (layer "B.Cu") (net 4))
 (segment (start 70.077 49.53) (end 70.104 49.557) (width 0.2) (layer "B.Cu") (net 4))
 (segment (start 58.6 46.6) (end 58.6 45.667) (width 0.2) (layer "B.Cu") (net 4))
 (segment (start 60.96 42.545) (end 60.96 46.482) (width 0.2) (layer "B.Cu") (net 4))
 (segment (start 67.31 49.53) (end 70.077 49.53) (width 0.2) (layer "B.Cu") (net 4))
 (segment (start 64.7645 40.828) (end 64.7645 41.722) (width 0.2) (layer "F.Cu") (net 3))
 (segment (start 65.614 43.2405) (end 66.802 44.4285) (width 1.5) (layer "F.Cu") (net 3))
 (segment (start 69.215 44.9155) (end 69.469 44.6615) (width 1.5) (layer "F.Cu") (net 3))
 (segment (start 67.564 44.7045) (end 67.607 44.6615) (width 1.5) (layer "F.Cu") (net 3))
 (segment (start 63.246 43.2405) (end 65.614 43.2405) (width 1.5) (layer "F.Cu") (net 3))
 (segment (start 67.078 44.7045) (end 67.564 44.7045) (width 1.5) (layer "F.Cu") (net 3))
 (segment (start 66.802 44.4285) (end 67.078 44.7045) (width 1.5) (layer "F.Cu") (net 3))
 (segment (start 69.215 46.2065) (end 69.215 44.9155) (width 1.5) (layer "F.Cu") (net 3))
 (segment (start 67.607 44.6615) (end 69.469 44.6615) (width 1.5) (layer "F.Cu") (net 3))
 (segment (start 64.7645 41.722) (end 63.246 43.2405) (width 0.2) (layer "F.Cu") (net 3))
 (segment (start 61.214 36.703) (end 69.85 36.703) (width 0.2) (layer "F.Cu") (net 8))
 (segment (start 60.325 37.592) (end 61.214 36.703) (width 0.2) (layer "F.Cu") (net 8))
 (segment (start 69.85 36.703) (end 71.247 38.1) (width 0.2) (layer "F.Cu") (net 8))
 (via (at 71.247 38.1) (size 0.6) (drill 0.3) (layers "F.Cu" "B.Cu") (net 8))
 (via (at 60.325 37.592) (size 0.6) (drill 0.3) (layers "F.Cu" "B.Cu") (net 8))
 (segment (start 71.247 38.1) (end 72.152 38.1) (width 0.2) (layer "B.Cu") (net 8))
 (segment (start 58.674 39.243) (end 60.325 37.592) (width 0.2) (layer "B.Cu") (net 8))
 (segment (start 72.009 38.243) (end 72.009 39.39537) (width 0.2) (layer "B.Cu") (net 8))
 (segment (start 72.009 39.39537) (end 72.62963 40.016) (width 0.2) (layer "B.Cu") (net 8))
 (segment (start 72.914 37.338) (end 72.009 38.243) (width 0.2) (layer "B.Cu") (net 8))
 (segment (start 72.62963 40.016) (end 73.287 40.016) (width 0.2) (layer "B.Cu") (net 8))
 (segment (start 72.152 38.1) (end 72.914 37.338) (width 0.2) (layer "B.Cu") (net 8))
 (segment (start 58.674 40.513) (end 58.674 39.243) (width 0.2) (layer "B.Cu") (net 8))
 (segment (start 74.422 40.132) (end 74.419 40.129) (width 0.8) (layer "F.Cu") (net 1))
 (segment (start 74.419 40.129) (end 74.419 37.846) (width 1.5) (layer "F.Cu") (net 1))
 (segment (start 74.419 37.846) (end 74.038 37.465) (width 0.8) (layer "F.Cu") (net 1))
 (segment (start 74.419 44.834) (end 74.419 47.625) (width 1.5) (layer "F.Cu") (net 2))
 (segment (start 74.422 44.831) (end 74.419 44.834) (width 0.8) (layer "F.Cu") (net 2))
 (segment (start 74.419 47.625) (end 74.038 48.006) (width 0.8) (layer "F.Cu") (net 2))
 (segment (start 71.031003 39.116) (end 70.739 39.116) (width 0.2) (layer "F.Cu") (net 13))
 (segment (start 69.723 38.1) (end 69.088 38.1) (width 0.2) (layer "F.Cu") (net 13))
 (segment (start 71.247 38.900003) (end 71.031003 39.116) (width 0.2) (layer "F.Cu") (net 13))
 (segment (start 70.739 39.116) (end 69.723 38.1) (width 0.2) (layer "F.Cu") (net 13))
 (via (at 71.247 38.900003) (size 0.6) (drill 0.3) (layers "F.Cu" "B.Cu") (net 13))
 (via (at 69.088 38.1) (size 0.6) (drill 0.3) (layers "F.Cu" "B.Cu") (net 13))
 (segment (start 72.558 41.316) (end 73.287 41.316) (width 0.2) (layer "B.Cu") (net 13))
 (segment (start 71.247 38.900003) (end 71.247 40.005) (width 0.2) (layer "B.Cu") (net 13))
 (segment (start 71.247 40.005) (end 72.558 41.316) (width 0.2) (layer "B.Cu") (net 13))
 (segment (start 69.088 38.1) (end 67.437 36.449) (width 0.2) (layer "B.Cu") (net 13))
 (segment (start 64.897 36.449) (end 65.312 36.864) (width 0.2) (layer "B.Cu") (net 14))
 (segment (start 65.312 39.872943) (end 66.105057 40.666) (width 0.2) (layer "B.Cu") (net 14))
 (segment (start 65.312 36.864) (end 65.312 39.872943) (width 0.2) (layer "B.Cu") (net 14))
 (segment (start 66.105057 40.666) (end 67.562 40.666) (width 0.2) (layer "B.Cu") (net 14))
 (segment (start 68.834 44.704) (end 68.834 43.800501) (width 0.2) (layer "B.Cu") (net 15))
 (segment (start 68.834 43.800501) (end 68.299499 43.266) (width 0.2) (layer "B.Cu") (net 15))
 (segment (start 64.774 45.216) (end 67.562 45.216) (width 0.2) (layer "B.Cu") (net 15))
 (segment (start 68.322 45.216) (end 68.834 44.704) (width 0.2) (layer "B.Cu") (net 15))
 (segment (start 63.881 44.323) (end 64.774 45.216) (width 0.2) (layer "B.Cu") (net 15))
 (segment (start 68.299499 43.266) (end 67.562 43.266) (width 0.2) (layer "B.Cu") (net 15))
 (segment (start 67.562 45.216) (end 68.322 45.216) (width 0.2) (layer "B.Cu") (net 15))
 (segment (start 66.664 44.566) (end 63.881 41.783) (width 0.2) (layer "B.Cu") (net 22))
 (segment (start 67.562 44.566) (end 66.664 44.566) (width 0.2) (layer "B.Cu") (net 22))
 (segment (start 62.4895 38.928) (end 63.185 38.928) (width 0.2) (layer "F.Cu") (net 5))
 (segment (start 63.881 39.624) (end 65.913 39.624) (width 0.2) (layer "F.Cu") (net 5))
 (segment (start 63.185 38.928) (end 63.881 39.624) (width 0.2) (layer "F.Cu") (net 5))
 (via (at 65.913 39.624) (size 0.6) (drill 0.3) (layers "F.Cu" "B.Cu") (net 5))
 (segment (start 66.171 39.366) (end 65.913 39.624) (width 0.2) (layer "B.Cu") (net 5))
 (segment (start 67.562 39.366) (end 66.171 39.366) (width 0.2) (layer "B.Cu") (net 5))
 (segment (start 67.0445 41.3905) (end 67.564 41.91) (width 0.2) (layer "F.Cu") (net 10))
 (segment (start 67.564 41.91) (end 69.469 41.91) (width 0.2) (layer "F.Cu") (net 10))
 (segment (start 66.031876 41.3905) (end 67.0445 41.3905) (width 0.2) (layer "F.Cu") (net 10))
 (via (at 66.031876 41.3905) (size 0.6) (drill 0.3) (layers "F.Cu" "B.Cu") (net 10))
 (segment (start 66.619 42.616) (end 66.04 42.037) (width 0.2) (layer "B.Cu") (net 10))
 (segment (start 66.04 41.398624) (end 66.031876 41.3905) (width 0.2) (layer "B.Cu") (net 10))
 (segment (start 67.562 42.616) (end 66.619 42.616) (width 0.2) (layer "B.Cu") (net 10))
 (segment (start 66.04 42.037) (end 66.04 41.398624) (width 0.2) (layer "B.Cu") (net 10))
 (segment (start 65.400126 41.9905) (end 66.3745 41.9905) (width 0.2) (layer "F.Cu") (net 11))
 (segment (start 66.3745 41.9905) (end 67.564 43.18) (width 0.2) (layer "F.Cu") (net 11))
 (segment (start 67.564 43.18) (end 69.469 43.18) (width 0.2) (layer "F.Cu") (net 11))
 (via (at 65.400126 41.9905) (size 0.6) (drill 0.3) (layers "F.Cu" "B.Cu") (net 11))
 (segment (start 67.562 43.916) (end 66.824501 43.916) (width 0.2) (layer "B.Cu") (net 11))
 (segment (start 66.824501 43.916) (end 65.405 42.496499) (width 0.2) (layer "B.Cu") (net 11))
 (segment (start 65.405 42.496499) (end 65.405 41.995374) (width 0.2) (layer "B.Cu") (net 11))
 (segment (start 65.405 41.995374) (end 65.400126 41.9905) (width 0.2) (layer "B.Cu") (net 11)))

